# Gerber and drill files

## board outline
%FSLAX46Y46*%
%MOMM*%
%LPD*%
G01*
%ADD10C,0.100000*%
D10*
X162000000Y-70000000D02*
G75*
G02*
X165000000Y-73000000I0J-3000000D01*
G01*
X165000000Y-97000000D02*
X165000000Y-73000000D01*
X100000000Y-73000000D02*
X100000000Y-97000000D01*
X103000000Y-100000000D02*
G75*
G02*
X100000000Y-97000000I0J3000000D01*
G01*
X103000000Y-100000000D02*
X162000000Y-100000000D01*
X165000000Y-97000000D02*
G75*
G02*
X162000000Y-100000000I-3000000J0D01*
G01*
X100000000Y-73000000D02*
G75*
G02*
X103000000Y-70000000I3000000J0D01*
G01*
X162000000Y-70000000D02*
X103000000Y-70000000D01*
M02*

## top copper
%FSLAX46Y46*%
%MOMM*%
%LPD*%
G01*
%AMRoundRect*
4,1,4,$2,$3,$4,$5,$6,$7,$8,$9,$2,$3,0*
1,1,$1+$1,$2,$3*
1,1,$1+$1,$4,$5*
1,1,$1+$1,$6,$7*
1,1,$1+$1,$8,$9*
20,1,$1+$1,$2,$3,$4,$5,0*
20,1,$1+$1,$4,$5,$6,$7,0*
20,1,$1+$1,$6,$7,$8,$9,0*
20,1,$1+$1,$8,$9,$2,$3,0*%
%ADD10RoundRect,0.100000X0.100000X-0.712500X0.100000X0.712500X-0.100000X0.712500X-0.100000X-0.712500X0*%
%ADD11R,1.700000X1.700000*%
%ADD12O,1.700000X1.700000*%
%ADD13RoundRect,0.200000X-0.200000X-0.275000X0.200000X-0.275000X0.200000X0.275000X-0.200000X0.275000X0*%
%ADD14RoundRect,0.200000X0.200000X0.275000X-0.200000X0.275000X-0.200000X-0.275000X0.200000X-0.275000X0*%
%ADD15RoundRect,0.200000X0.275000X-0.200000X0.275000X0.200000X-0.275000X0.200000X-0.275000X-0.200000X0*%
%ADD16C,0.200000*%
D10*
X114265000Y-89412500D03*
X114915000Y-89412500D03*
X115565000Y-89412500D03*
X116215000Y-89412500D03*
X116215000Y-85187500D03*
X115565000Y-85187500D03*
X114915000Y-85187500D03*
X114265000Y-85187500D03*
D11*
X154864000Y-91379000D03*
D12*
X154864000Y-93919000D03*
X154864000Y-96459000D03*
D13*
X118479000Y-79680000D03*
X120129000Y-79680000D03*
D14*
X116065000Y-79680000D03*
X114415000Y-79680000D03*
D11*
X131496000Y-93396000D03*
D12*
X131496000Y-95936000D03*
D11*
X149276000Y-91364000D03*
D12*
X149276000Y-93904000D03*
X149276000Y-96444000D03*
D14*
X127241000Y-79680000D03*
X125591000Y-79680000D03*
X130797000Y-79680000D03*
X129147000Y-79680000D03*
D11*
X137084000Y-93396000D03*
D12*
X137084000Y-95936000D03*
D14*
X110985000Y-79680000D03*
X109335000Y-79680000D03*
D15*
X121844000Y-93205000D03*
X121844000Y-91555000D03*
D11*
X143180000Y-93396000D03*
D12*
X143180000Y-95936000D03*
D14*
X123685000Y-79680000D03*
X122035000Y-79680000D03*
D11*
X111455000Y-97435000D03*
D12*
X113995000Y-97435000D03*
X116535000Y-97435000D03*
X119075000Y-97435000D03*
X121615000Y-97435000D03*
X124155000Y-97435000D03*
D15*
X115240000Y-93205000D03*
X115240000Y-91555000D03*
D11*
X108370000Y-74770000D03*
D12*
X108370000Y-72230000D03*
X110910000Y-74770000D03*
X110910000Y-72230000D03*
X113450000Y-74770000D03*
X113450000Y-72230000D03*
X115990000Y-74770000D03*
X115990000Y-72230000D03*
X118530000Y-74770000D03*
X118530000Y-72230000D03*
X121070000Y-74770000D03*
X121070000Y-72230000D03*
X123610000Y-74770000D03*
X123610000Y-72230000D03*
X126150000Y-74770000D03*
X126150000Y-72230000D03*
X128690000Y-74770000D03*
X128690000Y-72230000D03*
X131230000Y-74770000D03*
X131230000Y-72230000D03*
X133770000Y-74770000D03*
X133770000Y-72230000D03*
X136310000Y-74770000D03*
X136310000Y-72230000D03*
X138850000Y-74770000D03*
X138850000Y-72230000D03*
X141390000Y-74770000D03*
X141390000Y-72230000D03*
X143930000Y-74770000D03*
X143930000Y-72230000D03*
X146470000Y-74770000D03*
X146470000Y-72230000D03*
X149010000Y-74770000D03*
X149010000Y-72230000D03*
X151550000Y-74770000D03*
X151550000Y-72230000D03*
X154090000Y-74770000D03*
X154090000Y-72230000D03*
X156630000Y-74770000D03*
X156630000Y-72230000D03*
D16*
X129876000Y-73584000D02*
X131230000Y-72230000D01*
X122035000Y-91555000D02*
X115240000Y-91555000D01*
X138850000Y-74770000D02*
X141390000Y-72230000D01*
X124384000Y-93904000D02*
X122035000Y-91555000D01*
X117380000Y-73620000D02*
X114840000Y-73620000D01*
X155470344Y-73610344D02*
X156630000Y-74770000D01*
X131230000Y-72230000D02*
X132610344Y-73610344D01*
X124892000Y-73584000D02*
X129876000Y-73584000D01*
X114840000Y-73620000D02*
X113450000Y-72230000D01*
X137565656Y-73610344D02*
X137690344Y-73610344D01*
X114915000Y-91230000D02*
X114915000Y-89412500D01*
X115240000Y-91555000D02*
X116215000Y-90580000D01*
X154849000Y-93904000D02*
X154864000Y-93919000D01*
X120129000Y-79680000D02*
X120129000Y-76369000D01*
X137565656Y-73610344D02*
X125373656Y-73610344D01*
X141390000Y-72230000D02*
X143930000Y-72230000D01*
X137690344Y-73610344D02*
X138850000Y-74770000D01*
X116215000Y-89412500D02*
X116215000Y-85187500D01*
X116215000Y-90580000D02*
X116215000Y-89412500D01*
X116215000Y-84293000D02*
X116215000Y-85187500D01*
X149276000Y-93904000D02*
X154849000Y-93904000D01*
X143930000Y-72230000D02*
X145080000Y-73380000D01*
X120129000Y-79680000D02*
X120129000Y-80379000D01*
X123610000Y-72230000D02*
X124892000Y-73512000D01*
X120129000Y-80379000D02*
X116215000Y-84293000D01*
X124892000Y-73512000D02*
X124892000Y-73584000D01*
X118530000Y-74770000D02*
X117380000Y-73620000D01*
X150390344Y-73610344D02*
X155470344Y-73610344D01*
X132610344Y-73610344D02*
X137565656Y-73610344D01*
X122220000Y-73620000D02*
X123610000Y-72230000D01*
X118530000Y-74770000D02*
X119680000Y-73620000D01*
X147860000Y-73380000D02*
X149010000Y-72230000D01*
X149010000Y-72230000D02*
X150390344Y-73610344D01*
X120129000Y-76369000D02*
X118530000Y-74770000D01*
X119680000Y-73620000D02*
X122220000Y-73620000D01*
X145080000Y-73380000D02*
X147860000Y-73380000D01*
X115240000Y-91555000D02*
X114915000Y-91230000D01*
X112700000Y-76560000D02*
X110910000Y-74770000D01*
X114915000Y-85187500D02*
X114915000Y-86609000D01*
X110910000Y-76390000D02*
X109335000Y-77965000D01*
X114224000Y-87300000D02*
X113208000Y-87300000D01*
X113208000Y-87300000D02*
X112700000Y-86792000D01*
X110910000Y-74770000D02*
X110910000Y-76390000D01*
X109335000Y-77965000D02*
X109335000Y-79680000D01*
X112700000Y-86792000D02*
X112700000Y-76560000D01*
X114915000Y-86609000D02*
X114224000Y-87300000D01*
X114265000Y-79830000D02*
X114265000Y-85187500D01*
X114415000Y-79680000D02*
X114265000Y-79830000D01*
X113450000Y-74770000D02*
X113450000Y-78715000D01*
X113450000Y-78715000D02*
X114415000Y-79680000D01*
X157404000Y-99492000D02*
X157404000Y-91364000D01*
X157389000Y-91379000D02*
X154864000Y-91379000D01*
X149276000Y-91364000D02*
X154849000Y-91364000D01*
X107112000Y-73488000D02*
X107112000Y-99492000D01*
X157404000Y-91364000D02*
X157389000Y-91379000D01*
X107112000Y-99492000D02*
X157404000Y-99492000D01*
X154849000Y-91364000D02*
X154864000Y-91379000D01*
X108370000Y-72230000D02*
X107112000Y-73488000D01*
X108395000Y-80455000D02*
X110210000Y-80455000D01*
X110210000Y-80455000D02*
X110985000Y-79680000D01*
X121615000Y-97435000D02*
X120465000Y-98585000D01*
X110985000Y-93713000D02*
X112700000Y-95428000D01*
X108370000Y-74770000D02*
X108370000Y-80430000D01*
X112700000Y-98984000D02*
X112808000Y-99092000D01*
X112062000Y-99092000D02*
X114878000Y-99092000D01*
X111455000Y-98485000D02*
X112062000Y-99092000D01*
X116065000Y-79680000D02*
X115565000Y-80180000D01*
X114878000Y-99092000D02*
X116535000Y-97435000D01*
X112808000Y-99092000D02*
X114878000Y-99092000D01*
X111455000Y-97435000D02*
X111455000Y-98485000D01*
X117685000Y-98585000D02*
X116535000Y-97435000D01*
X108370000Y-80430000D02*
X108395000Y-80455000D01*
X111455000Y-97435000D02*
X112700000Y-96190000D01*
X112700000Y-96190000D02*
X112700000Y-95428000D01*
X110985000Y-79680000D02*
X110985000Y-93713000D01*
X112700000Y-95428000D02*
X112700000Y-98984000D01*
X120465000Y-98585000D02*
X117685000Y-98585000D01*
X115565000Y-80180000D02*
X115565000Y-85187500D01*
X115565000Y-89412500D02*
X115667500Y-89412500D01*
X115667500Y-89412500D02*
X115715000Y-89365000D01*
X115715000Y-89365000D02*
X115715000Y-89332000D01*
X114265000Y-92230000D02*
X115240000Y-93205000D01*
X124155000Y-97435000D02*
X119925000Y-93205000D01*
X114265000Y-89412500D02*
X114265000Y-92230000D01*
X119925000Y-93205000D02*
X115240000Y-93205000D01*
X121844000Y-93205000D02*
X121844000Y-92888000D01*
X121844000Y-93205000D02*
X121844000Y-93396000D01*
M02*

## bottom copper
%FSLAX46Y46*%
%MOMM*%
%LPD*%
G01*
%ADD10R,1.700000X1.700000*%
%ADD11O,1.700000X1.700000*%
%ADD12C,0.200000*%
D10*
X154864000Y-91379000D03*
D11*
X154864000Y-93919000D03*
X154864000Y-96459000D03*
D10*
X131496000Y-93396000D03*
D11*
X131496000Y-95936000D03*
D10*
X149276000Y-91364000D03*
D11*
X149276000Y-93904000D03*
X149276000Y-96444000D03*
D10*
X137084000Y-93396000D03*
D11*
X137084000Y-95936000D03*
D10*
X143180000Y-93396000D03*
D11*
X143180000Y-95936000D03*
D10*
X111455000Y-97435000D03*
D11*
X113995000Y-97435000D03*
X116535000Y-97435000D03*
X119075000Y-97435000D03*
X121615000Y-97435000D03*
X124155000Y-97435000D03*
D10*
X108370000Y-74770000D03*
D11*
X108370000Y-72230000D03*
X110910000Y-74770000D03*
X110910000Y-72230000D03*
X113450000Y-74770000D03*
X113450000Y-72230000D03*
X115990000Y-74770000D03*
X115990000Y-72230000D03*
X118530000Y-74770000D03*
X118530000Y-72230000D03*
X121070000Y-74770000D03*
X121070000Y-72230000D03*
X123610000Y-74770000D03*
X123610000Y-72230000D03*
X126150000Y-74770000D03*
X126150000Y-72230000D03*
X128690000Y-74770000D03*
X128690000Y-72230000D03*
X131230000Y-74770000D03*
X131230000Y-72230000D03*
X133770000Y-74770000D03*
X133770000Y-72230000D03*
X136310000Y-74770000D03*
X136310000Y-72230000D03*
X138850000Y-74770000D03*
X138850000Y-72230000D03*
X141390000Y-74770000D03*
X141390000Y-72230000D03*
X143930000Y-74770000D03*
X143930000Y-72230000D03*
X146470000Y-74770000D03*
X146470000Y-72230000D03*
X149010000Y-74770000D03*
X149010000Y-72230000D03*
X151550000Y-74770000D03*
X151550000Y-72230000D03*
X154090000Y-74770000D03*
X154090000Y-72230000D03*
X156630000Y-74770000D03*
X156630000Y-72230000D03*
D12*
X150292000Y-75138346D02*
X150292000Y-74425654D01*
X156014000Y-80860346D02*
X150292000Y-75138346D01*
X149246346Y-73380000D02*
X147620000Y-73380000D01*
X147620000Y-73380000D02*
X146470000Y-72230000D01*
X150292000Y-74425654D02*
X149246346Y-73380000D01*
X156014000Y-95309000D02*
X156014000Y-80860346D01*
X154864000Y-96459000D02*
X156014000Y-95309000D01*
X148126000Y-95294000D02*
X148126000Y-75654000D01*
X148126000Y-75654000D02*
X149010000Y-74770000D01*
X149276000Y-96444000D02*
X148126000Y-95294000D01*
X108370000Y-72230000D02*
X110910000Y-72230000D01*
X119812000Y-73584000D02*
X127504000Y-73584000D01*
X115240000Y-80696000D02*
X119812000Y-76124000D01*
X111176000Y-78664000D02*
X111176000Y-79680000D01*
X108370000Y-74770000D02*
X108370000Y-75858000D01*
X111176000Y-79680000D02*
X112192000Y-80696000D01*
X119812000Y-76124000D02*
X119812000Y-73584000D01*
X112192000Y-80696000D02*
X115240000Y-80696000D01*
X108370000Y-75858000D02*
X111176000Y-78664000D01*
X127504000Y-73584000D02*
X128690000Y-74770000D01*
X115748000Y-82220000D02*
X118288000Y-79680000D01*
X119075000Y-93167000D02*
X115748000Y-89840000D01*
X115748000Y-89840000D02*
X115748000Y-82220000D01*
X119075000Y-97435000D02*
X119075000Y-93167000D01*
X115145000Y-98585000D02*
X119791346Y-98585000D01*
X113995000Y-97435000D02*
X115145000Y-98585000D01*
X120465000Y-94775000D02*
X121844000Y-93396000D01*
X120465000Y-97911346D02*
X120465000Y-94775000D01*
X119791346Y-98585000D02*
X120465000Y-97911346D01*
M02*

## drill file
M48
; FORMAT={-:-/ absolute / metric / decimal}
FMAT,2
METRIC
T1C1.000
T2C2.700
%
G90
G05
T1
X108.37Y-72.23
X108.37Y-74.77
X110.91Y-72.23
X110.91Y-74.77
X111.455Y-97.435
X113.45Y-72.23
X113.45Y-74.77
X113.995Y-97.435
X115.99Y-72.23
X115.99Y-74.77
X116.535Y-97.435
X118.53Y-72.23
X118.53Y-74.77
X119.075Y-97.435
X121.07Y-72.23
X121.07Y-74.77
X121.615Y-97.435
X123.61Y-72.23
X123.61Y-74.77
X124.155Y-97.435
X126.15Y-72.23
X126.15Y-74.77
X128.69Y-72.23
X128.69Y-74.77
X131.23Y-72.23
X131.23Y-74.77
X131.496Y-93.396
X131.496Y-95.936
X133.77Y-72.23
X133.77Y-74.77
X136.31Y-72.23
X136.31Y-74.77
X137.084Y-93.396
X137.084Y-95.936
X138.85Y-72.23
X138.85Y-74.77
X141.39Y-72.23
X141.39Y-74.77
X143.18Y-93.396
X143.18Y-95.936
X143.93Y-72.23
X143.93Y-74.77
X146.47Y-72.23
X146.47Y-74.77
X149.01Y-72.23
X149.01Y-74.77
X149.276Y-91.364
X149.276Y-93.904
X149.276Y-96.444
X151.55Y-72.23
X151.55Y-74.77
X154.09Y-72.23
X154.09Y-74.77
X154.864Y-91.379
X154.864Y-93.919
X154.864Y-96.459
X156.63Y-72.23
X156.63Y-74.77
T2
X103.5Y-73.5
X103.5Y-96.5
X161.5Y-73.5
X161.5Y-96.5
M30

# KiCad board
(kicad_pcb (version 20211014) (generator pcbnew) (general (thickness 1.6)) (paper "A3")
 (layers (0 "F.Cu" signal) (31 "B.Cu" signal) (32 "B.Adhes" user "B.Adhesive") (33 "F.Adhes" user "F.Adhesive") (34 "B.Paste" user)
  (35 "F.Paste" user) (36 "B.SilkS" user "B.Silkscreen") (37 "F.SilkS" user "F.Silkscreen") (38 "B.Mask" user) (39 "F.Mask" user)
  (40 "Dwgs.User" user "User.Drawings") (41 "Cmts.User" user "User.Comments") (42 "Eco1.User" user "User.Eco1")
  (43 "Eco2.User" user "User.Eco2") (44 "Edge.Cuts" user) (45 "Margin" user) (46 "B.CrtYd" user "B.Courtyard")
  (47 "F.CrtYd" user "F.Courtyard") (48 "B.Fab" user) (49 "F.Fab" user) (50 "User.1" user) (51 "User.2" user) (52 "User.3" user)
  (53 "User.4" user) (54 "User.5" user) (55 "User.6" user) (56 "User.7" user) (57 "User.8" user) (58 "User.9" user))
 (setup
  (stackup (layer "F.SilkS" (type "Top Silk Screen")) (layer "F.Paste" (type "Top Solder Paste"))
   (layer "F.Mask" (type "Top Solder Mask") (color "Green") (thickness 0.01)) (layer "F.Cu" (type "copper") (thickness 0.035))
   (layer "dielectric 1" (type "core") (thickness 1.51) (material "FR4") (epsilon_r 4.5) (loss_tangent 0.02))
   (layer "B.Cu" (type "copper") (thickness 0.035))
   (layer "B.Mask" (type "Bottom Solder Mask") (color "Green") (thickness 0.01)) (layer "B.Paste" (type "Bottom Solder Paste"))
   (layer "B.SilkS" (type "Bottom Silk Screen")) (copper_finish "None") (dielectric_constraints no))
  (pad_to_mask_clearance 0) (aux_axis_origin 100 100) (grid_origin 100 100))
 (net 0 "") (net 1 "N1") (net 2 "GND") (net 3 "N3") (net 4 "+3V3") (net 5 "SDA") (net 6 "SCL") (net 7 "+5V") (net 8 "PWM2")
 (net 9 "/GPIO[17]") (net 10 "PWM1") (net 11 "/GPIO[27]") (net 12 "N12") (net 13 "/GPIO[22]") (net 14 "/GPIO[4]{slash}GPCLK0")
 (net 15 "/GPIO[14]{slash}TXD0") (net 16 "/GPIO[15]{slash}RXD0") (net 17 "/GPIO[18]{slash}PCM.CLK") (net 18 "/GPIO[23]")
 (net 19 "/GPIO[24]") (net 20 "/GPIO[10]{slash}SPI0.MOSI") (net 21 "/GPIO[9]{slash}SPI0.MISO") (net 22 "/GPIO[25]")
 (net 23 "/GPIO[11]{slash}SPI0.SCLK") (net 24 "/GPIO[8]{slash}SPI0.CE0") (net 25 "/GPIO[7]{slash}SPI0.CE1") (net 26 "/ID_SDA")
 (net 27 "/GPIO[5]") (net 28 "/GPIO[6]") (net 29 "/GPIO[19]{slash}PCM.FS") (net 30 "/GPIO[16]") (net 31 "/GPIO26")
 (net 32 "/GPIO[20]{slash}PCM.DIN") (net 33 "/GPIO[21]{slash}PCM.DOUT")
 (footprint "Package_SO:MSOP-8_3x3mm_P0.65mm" (layer "F.Cu") (at 115.24 87.3 90)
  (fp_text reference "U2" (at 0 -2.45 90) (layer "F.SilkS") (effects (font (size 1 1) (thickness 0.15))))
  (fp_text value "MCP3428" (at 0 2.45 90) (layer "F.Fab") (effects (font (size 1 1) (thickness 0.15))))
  (pad "1" smd roundrect (at -2.1125 -0.975 90) (size 1.625 0.4) (layers "F.Cu" "F.Paste" "F.Mask") (roundrect_rratio 0.25) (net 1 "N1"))
  (pad "2" smd roundrect (at -2.1125 -0.325 90) (size 1.625 0.4) (layers "F.Cu" "F.Paste" "F.Mask") (roundrect_rratio 0.25) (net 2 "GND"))
  (pad "3" smd roundrect (at -2.1125 0.325 90) (size 1.625 0.4) (layers "F.Cu" "F.Paste" "F.Mask") (roundrect_rratio 0.25) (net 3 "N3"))
  (pad "4" smd roundrect (at -2.1125 0.975 90) (size 1.625 0.4) (layers "F.Cu" "F.Paste" "F.Mask") (roundrect_rratio 0.25) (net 2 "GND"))
  (pad "5" smd roundrect (at 2.1125 0.975 90) (size 1.625 0.4) (layers "F.Cu" "F.Paste" "F.Mask") (roundrect_rratio 0.25) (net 2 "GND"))
  (pad "6" smd roundrect (at 2.1125 0.325 90) (size 1.625 0.4) (layers "F.Cu" "F.Paste" "F.Mask") (roundrect_rratio 0.25) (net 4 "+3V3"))
  (pad "7" smd roundrect (at 2.1125 -0.325 90) (size 1.625 0.4) (layers "F.Cu" "F.Paste" "F.Mask") (roundrect_rratio 0.25) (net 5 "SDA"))
  (pad "8" smd roundrect (at 2.1125 -0.975 90) (size 1.625 0.4) (layers "F.Cu" "F.Paste" "F.Mask") (roundrect_rratio 0.25) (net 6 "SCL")))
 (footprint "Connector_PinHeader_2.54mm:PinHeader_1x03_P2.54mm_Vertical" (layer "F.Cu") (at 154.864 91.379)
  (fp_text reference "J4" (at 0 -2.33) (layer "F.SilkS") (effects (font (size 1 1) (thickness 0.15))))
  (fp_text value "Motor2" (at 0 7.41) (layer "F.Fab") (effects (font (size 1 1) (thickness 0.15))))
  (pad "1" thru_hole rect (at 0 0) (size 1.7 1.7) (drill 1) (layers *.Cu *.Mask) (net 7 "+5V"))
  (pad "2" thru_hole oval (at 0 2.54) (size 1.7 1.7) (drill 1) (layers *.Cu *.Mask) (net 2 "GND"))
  (pad "3" thru_hole oval (at 0 5.08) (size 1.7 1.7) (drill 1) (layers *.Cu *.Mask) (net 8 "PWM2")))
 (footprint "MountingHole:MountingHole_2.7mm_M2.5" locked (layer "F.Cu") (at 161.5 73.5)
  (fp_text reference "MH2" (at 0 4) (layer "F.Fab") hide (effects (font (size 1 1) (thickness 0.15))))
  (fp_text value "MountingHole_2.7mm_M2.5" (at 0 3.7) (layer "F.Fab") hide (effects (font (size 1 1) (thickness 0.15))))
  (pad "" np_thru_hole circle locked (at 0 0) (size 2.7 2.7) (drill 2.7) (layers *.Cu *.Mask)))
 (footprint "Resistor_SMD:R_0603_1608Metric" (layer "F.Cu") (at 119.304 79.68)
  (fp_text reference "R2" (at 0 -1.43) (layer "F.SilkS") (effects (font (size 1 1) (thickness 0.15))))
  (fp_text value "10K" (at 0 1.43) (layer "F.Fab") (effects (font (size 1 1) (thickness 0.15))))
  (pad "1" smd roundrect (at -0.825 0) (size 0.8 0.95) (layers "F.Cu" "F.Paste" "F.Mask") (roundrect_rratio 0.25) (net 3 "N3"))
  (pad "2" smd roundrect (at 0.825 0) (size 0.8 0.95) (layers "F.Cu" "F.Paste" "F.Mask") (roundrect_rratio 0.25) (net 2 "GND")))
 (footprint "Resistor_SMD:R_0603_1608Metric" (layer "F.Cu") (at 115.24 79.68 180)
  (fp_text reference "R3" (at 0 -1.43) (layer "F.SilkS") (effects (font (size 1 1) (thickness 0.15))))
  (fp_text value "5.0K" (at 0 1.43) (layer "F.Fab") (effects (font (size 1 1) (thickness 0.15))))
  (pad "1" smd roundrect (at -0.825 0 180) (size 0.8 0.95) (layers "F.Cu" "F.Paste" "F.Mask") (roundrect_rratio 0.25) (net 4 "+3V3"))
  (pad "2" smd roundrect (at 0.825 0 180) (size 0.8 0.95) (layers "F.Cu" "F.Paste" "F.Mask") (roundrect_rratio 0.25) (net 6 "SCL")))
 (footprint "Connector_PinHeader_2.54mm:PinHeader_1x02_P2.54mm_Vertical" (layer "F.Cu") (at 131.496 93.396)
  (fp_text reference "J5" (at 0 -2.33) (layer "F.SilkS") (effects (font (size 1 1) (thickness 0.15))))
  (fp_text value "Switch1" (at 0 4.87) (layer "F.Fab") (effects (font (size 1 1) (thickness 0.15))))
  (pad "1" thru_hole rect (at 0 0) (size 1.7 1.7) (drill 1) (layers *.Cu *.Mask) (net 4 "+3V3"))
  (pad "2" thru_hole oval (at 0 2.54) (size 1.7 1.7) (drill 1) (layers *.Cu *.Mask) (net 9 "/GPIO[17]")))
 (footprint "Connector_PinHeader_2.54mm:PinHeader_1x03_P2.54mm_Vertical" (layer "F.Cu") (at 149.276 91.364)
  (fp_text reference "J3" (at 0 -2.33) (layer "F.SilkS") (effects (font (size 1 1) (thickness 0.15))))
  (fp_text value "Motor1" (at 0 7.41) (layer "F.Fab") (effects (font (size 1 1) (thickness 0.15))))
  (pad "1" thru_hole rect (at 0 0) (size 1.7 1.7) (drill 1) (layers *.Cu *.Mask) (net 7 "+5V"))
  (pad "2" thru_hole oval (at 0 2.54) (size 1.7 1.7) (drill 1) (layers *.Cu *.Mask) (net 2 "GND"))
  (pad "3" thru_hole oval (at 0 5.08) (size 1.7 1.7) (drill 1) (layers *.Cu *.Mask) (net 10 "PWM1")))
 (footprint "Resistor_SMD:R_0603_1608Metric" (layer "F.Cu") (at 126.416 79.68 180)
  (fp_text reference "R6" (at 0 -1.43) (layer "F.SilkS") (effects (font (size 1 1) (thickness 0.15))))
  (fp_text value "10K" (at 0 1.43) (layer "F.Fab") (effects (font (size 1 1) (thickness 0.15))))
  (pad "1" smd roundrect (at -0.825 0 180) (size 0.8 0.95) (layers "F.Cu" "F.Paste" "F.Mask") (roundrect_rratio 0.25) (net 9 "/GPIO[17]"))
  (pad "2" smd roundrect (at 0.825 0 180) (size 0.8 0.95) (layers "F.Cu" "F.Paste" "F.Mask") (roundrect_rratio 0.25) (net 2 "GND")))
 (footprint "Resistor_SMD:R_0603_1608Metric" (layer "F.Cu") (at 129.972 79.68 180)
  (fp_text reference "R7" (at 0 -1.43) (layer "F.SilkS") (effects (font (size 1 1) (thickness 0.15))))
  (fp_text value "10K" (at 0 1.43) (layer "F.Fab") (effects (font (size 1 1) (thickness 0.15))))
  (pad "1" smd roundrect (at -0.825 0 180) (size 0.8 0.95) (layers "F.Cu" "F.Paste" "F.Mask") (roundrect_rratio 0.25) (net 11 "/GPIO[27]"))
  (pad "2" smd roundrect (at 0.825 0 180) (size 0.8 0.95) (layers "F.Cu" "F.Paste" "F.Mask") (roundrect_rratio 0.25) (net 2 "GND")))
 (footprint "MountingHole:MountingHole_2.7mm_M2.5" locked (layer "F.Cu") (at 103.5 96.5)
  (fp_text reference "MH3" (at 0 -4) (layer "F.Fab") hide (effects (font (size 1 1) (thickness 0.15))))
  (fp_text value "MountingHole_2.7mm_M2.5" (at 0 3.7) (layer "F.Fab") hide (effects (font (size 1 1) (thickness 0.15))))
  (pad "" np_thru_hole circle locked (at 0 0) (size 2.7 2.7) (drill 2.7) (layers *.Cu *.Mask)))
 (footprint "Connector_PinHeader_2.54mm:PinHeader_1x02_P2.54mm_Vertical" (layer "F.Cu") (at 137.084 93.396)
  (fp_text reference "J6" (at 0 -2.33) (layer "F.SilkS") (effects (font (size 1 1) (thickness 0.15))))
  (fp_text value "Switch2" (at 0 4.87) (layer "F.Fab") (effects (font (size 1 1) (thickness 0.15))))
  (pad "1" thru_hole rect (at 0 0) (size 1.7 1.7) (drill 1) (layers *.Cu *.Mask) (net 4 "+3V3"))
  (pad "2" thru_hole oval (at 0 2.54) (size 1.7 1.7) (drill 1) (layers *.Cu *.Mask) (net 11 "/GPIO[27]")))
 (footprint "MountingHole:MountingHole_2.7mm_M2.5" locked (layer "F.Cu") (at 103.5 73.5)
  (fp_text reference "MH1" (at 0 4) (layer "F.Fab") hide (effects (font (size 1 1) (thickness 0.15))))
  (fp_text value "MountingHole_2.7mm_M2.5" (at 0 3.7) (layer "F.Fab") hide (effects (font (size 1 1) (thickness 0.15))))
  (pad "" np_thru_hole circle locked (at 0 0) (size 2.7 2.7) (drill 2.7) (layers *.Cu *.Mask)))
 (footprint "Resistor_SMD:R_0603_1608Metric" (layer "F.Cu") (at 110.16 79.68 180)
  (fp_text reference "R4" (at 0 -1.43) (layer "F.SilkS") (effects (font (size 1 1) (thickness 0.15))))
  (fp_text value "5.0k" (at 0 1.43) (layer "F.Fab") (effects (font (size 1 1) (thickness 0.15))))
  (pad "1" smd roundrect (at -0.825 0 180) (size 0.8 0.95) (layers "F.Cu" "F.Paste" "F.Mask") (roundrect_rratio 0.25) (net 4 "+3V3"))
  (pad "2" smd roundrect (at 0.825 0 180) (size 0.8 0.95) (layers "F.Cu" "F.Paste" "F.Mask") (roundrect_rratio 0.25) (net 5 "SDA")))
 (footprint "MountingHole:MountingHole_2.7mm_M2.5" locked (layer "F.Cu") (at 161.5 96.5)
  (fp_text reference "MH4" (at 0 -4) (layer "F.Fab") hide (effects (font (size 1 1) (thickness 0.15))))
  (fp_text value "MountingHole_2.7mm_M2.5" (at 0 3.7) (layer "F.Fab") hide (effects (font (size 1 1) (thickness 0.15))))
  (pad "" np_thru_hole circle locked (at 0 0) (size 2.7 2.7) (drill 2.7) (layers *.Cu *.Mask)))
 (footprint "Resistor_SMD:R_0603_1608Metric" (layer "F.Cu") (at 121.844 92.38 90)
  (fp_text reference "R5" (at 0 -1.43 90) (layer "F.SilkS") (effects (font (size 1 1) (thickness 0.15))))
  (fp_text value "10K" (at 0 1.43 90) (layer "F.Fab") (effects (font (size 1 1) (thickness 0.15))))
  (pad "1" smd roundrect (at -0.825 0 90) (size 0.8 0.95) (layers "F.Cu" "F.Paste" "F.Mask") (roundrect_rratio 0.25) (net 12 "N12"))
  (pad "2" smd roundrect (at 0.825 0 90) (size 0.8 0.95) (layers "F.Cu" "F.Paste" "F.Mask") (roundrect_rratio 0.25) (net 2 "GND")))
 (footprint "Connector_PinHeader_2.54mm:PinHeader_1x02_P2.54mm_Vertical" (layer "F.Cu") (at 143.18 93.396)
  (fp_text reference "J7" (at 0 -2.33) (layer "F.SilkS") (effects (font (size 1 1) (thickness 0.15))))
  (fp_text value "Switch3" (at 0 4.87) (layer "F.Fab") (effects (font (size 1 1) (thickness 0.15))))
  (pad "1" thru_hole rect (at 0 0) (size 1.7 1.7) (drill 1) (layers *.Cu *.Mask) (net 4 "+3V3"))
  (pad "2" thru_hole oval (at 0 2.54) (size 1.7 1.7) (drill 1) (layers *.Cu *.Mask) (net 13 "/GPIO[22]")))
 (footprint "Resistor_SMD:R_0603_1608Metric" (layer "F.Cu") (at 122.86 79.68 180)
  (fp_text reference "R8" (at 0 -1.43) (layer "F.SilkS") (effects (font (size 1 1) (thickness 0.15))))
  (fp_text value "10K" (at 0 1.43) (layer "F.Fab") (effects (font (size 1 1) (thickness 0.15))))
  (pad "1" smd roundrect (at -0.825 0 180) (size 0.8 0.95) (layers "F.Cu" "F.Paste" "F.Mask") (roundrect_rratio 0.25) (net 13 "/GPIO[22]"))
  (pad "2" smd roundrect (at 0.825 0 180) (size 0.8 0.95) (layers "F.Cu" "F.Paste" "F.Mask") (roundrect_rratio 0.25) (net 2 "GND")))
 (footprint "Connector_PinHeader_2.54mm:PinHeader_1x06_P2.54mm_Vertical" (layer "F.Cu") (at 111.455 97.435 90)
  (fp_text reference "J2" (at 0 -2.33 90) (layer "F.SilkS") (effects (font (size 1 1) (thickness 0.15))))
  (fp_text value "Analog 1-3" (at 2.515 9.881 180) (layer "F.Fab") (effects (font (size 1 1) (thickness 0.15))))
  (pad "1" thru_hole rect (at 0 0 90) (size 1.7 1.7) (drill 1) (layers *.Cu *.Mask) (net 4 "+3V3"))
  (pad "2" thru_hole oval (at 0 2.54 90) (size 1.7 1.7) (drill 1) (layers *.Cu *.Mask) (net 12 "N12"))
  (pad "3" thru_hole oval (at 0 5.08 90) (size 1.7 1.7) (drill 1) (layers *.Cu *.Mask) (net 4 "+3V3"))
  (pad "4" thru_hole oval (at 0 7.62 90) (size 1.7 1.7) (drill 1) (layers *.Cu *.Mask) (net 3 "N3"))
  (pad "5" thru_hole oval (at 0 10.16 90) (size 1.7 1.7) (drill 1) (layers *.Cu *.Mask) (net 4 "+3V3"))
  (pad "6" thru_hole oval (at 0 12.7 90) (size 1.7 1.7) (drill 1) (layers *.Cu *.Mask) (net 1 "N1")))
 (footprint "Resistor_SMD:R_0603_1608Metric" (layer "F.Cu") (at 115.24 92.38 90)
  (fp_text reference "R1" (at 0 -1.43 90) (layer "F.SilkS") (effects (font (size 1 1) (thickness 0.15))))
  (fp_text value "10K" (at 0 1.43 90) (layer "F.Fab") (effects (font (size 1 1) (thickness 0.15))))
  (pad "1" smd roundrect (at -0.825 0 90) (size 0.8 0.95) (layers "F.Cu" "F.Paste" "F.Mask") (roundrect_rratio 0.25) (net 1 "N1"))
  (pad "2" smd roundrect (at 0.825 0 90) (size 0.8 0.95) (layers "F.Cu" "F.Paste" "F.Mask") (roundrect_rratio 0.25) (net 2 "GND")))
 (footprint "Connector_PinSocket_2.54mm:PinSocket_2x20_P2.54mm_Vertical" (layer "B.Cu") (at 108.37 74.77 -90)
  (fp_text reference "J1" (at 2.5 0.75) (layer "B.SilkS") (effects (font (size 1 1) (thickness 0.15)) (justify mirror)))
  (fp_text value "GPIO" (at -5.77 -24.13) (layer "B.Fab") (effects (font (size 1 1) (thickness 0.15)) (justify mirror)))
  (pad "1" thru_hole rect locked (at 0 0 270) (size 1.7 1.7) (drill 1) (layers *.Cu *.Mask) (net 4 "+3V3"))
  (pad "2" thru_hole oval locked (at -2.54 0 270) (size 1.7 1.7) (drill 1) (layers *.Cu *.Mask) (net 7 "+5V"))
  (pad "3" thru_hole oval locked (at 0 -2.54 270) (size 1.7 1.7) (drill 1) (layers *.Cu *.Mask) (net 5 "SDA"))
  (pad "4" thru_hole oval locked (at -2.54 -2.54 270) (size 1.7 1.7) (drill 1) (layers *.Cu *.Mask) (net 7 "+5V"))
  (pad "5" thru_hole oval locked (at 0 -5.08 270) (size 1.7 1.7) (drill 1) (layers *.Cu *.Mask) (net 6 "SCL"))
  (pad "6" thru_hole oval locked (at -2.54 -5.08 270) (size 1.7 1.7) (drill 1) (layers *.Cu *.Mask) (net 2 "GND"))
  (pad "7" thru_hole oval locked (at 0 -7.62 270) (size 1.7 1.7) (drill 1) (layers *.Cu *.Mask) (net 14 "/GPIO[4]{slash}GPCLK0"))
  (pad "8" thru_hole oval locked (at -2.54 -7.62 270) (size 1.7 1.7) (drill 1) (layers *.Cu *.Mask) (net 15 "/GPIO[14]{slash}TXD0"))
  (pad "9" thru_hole oval locked (at 0 -10.16 270) (size 1.7 1.7) (drill 1) (layers *.Cu *.Mask) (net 2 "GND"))
  (pad "10" thru_hole oval locked (at -2.54 -10.16 270) (size 1.7 1.7) (drill 1) (layers *.Cu *.Mask) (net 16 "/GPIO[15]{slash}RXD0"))
  (pad "11" thru_hole oval locked (at 0 -12.7 270) (size 1.7 1.7) (drill 1) (layers *.Cu *.Mask) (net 9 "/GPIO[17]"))
  (pad "12" thru_hole oval locked (at -2.54 -12.7 270) (size 1.7 1.7) (drill 1) (layers *.Cu *.Mask) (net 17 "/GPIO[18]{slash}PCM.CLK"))
  (pad "13" thru_hole oval locked (at 0 -15.24 270) (size 1.7 1.7) (drill 1) (layers *.Cu *.Mask) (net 11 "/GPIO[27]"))
  (pad "14" thru_hole oval locked (at -2.54 -15.24 270) (size 1.7 1.7) (drill 1) (layers *.Cu *.Mask) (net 2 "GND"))
  (pad "15" thru_hole oval locked (at 0 -17.78 270) (size 1.7 1.7) (drill 1) (layers *.Cu *.Mask) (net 13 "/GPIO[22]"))
  (pad "16" thru_hole oval locked (at -2.54 -17.78 270) (size 1.7 1.7) (drill 1) (layers *.Cu *.Mask) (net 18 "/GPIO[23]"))
  (pad "17" thru_hole oval locked (at 0 -20.32 270) (size 1.7 1.7) (drill 1) (layers *.Cu *.Mask) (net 4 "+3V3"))
  (pad "18" thru_hole oval locked (at -2.54 -20.32 270) (size 1.7 1.7) (drill 1) (layers *.Cu *.Mask) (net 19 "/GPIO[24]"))
  (pad "19" thru_hole oval locked (at 0 -22.86 270) (size 1.7 1.7) (drill 1) (layers *.Cu *.Mask) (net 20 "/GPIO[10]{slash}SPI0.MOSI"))
  (pad "20" thru_hole oval locked (at -2.54 -22.86 270) (size 1.7 1.7) (drill 1) (layers *.Cu *.Mask) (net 2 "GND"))
  (pad "21" thru_hole oval locked (at 0 -25.4 270) (size 1.7 1.7) (drill 1) (layers *.Cu *.Mask) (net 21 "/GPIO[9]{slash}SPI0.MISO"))
  (pad "22" thru_hole oval locked (at -2.54 -25.4 270) (size 1.7 1.7) (drill 1) (layers *.Cu *.Mask) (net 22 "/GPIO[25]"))
  (pad "23" thru_hole oval locked (at 0 -27.94 270) (size 1.7 1.7) (drill 1) (layers *.Cu *.Mask) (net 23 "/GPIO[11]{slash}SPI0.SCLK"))
  (pad "24" thru_hole oval locked (at -2.54 -27.94 270) (size 1.7 1.7) (drill 1) (layers *.Cu *.Mask) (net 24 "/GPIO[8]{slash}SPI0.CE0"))
  (pad "25" thru_hole oval locked (at 0 -30.48 270) (size 1.7 1.7) (drill 1) (layers *.Cu *.Mask) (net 2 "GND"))
  (pad "26" thru_hole oval locked (at -2.54 -30.48 270) (size 1.7 1.7) (drill 1) (layers *.Cu *.Mask) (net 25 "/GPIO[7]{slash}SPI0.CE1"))
  (pad "27" thru_hole oval locked (at 0 -33.02 270) (size 1.7 1.7) (drill 1) (layers *.Cu *.Mask) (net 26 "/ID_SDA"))
  (pad "28" thru_hole oval locked (at -2.54 -33.02 270) (size 1.7 1.7) (drill 1) (layers *.Cu *.Mask) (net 2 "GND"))
  (pad "29" thru_hole oval locked (at 0 -35.56 270) (size 1.7 1.7) (drill 1) (layers *.Cu *.Mask) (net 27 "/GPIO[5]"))
  (pad "30" thru_hole oval locked (at -2.54 -35.56 270) (size 1.7 1.7) (drill 1) (layers *.Cu *.Mask) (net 2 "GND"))
  (pad "31" thru_hole oval locked (at 0 -38.1 270) (size 1.7 1.7) (drill 1) (layers *.Cu *.Mask) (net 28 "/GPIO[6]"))
  (pad "32" thru_hole oval locked (at -2.54 -38.1 270) (size 1.7 1.7) (drill 1) (layers *.Cu *.Mask) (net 8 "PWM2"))
  (pad "33" thru_hole oval locked (at 0 -40.64 270) (size 1.7 1.7) (drill 1) (layers *.Cu *.Mask) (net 10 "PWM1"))
  (pad "34" thru_hole oval locked (at -2.54 -40.64 270) (size 1.7 1.7) (drill 1) (layers *.Cu *.Mask) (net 2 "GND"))
  (pad "35" thru_hole oval locked (at 0 -43.18 270) (size 1.7 1.7) (drill 1) (layers *.Cu *.Mask) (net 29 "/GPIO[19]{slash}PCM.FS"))
  (pad "36" thru_hole oval locked (at -2.54 -43.18 270) (size 1.7 1.7) (drill 1) (layers *.Cu *.Mask) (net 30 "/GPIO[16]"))
  (pad "37" thru_hole oval locked (at 0 -45.72 270) (size 1.7 1.7) (drill 1) (layers *.Cu *.Mask) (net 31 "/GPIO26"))
  (pad "38" thru_hole oval locked (at -2.54 -45.72 270) (size 1.7 1.7) (drill 1) (layers *.Cu *.Mask) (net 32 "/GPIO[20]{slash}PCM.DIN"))
  (pad "39" thru_hole oval locked (at 0 -48.26 270) (size 1.7 1.7) (drill 1) (layers *.Cu *.Mask) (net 2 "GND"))
  (pad "40" thru_hole oval locked (at -2.54 -48.26 270) (size 1.7 1.7) (drill 1) (layers *.Cu *.Mask) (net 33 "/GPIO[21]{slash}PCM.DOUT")))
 (gr_arc (start 162 70) (mid 164.12132 70.87868) (end 165 73) (layer "Edge.Cuts") (width 0.1))
 (gr_line (start 165 97) (end 165 73) (layer "Edge.Cuts") (width 0.1))
 (gr_line (start 100 73) (end 100 97) (layer "Edge.Cuts") (width 0.1))
 (gr_arc (start 103 100) (mid 100.87868 99.12132) (end 100 97) (layer "Edge.Cuts") (width 0.1))
 (gr_line (start 103 100) (end 162 100) (layer "Edge.Cuts") (width 0.1))
 (gr_arc (start 165 97) (mid 164.12132 99.12132) (end 162 100) (layer "Edge.Cuts") (width 0.1))
 (gr_arc (start 100 73) (mid 100.87868 70.87868) (end 103 70) (layer "Edge.Cuts") (width 0.1))
 (gr_line (start 162 70) (end 103 70) (layer "Edge.Cuts") (width 0.1))
 (segment (start 129.876 73.584) (end 131.23 72.23) (width 0.2) (layer "F.Cu") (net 2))
 (segment (start 122.035 91.555) (end 115.24 91.555) (width 0.2) (layer "F.Cu") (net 2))
 (segment (start 138.85 74.77) (end 141.39 72.23) (width 0.2) (layer "F.Cu") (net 2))
 (segment (start 124.384 93.904) (end 122.035 91.555) (width 0.2) (layer "F.Cu") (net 2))
 (segment (start 117.38 73.62) (end 114.84 73.62) (width 0.2) (layer "F.Cu") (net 2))
 (segment (start 155.470344 73.610344) (end 156.63 74.77) (width 0.2) (layer "F.Cu") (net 2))
 (segment (start 131.23 72.23) (end 132.610344 73.610344) (width 0.2) (layer "F.Cu") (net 2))
 (segment (start 124.892 73.584) (end 129.876 73.584) (width 0.2) (layer "F.Cu") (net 2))
 (segment (start 114.84 73.62) (end 113.45 72.23) (width 0.2) (layer "F.Cu") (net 2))
 (segment (start 137.565656 73.610344) (end 137.690344 73.610344) (width 0.2) (layer "F.Cu") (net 2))
 (segment (start 114.915 91.23) (end 114.915 89.4125) (width 0.2) (layer "F.Cu") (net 2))
 (segment (start 115.24 91.555) (end 116.215 90.58) (width 0.2) (layer "F.Cu") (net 2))
 (segment (start 154.849 93.904) (end 154.864 93.919) (width 0.2) (layer "F.Cu") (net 2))
 (segment (start 120.129 79.68) (end 120.129 76.369) (width 0.2) (layer "F.Cu") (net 2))
 (segment (start 137.565656 73.610344) (end 125.373656 73.610344) (width 0.2) (layer "F.Cu") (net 2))
 (segment (start 141.39 72.23) (end 143.93 72.23) (width 0.2) (layer "F.Cu") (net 2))
 (segment (start 137.690344 73.610344) (end 138.85 74.77) (width 0.2) (layer "F.Cu") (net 2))
 (segment (start 116.215 89.4125) (end 116.215 85.1875) (width 0.2) (layer "F.Cu") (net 2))
 (segment (start 116.215 90.58) (end 116.215 89.4125) (width 0.2) (layer "F.Cu") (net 2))
 (segment (start 116.215 84.293) (end 116.215 85.1875) (width 0.2) (layer "F.Cu") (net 2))
 (segment (start 149.276 93.904) (end 154.849 93.904) (width 0.2) (layer "F.Cu") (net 2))
 (segment (start 143.93 72.23) (end 145.08 73.38) (width 0.2) (layer "F.Cu") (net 2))
 (segment (start 120.129 79.68) (end 120.129 80.379) (width 0.2) (layer "F.Cu") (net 2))
 (segment (start 123.61 72.23) (end 124.892 73.512) (width 0.2) (layer "F.Cu") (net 2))
 (segment (start 120.129 80.379) (end 116.215 84.293) (width 0.2) (layer "F.Cu") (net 2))
 (segment (start 124.892 73.512) (end 124.892 73.584) (width 0.2) (layer "F.Cu") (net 2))
 (segment (start 118.53 74.77) (end 117.38 73.62) (width 0.2) (layer "F.Cu") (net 2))
 (segment (start 150.390344 73.610344) (end 155.470344 73.610344) (width 0.2) (layer "F.Cu") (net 2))
 (segment (start 132.610344 73.610344) (end 137.565656 73.610344) (width 0.2) (layer "F.Cu") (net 2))
 (segment (start 122.22 73.62) (end 123.61 72.23) (width 0.2) (layer "F.Cu") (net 2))
 (segment (start 118.53 74.77) (end 119.68 73.62) (width 0.2) (layer "F.Cu") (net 2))
 (segment (start 147.86 73.38) (end 149.01 72.23) (width 0.2) (layer "F.Cu") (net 2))
 (segment (start 149.01 72.23) (end 150.390344 73.610344) (width 0.2) (layer "F.Cu") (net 2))
 (segment (start 120.129 76.369) (end 118.53 74.77) (width 0.2) (layer "F.Cu") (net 2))
 (segment (start 119.68 73.62) (end 122.22 73.62) (width 0.2) (layer "F.Cu") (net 2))
 (segment (start 145.08 73.38) (end 147.86 73.38) (width 0.2) (layer "F.Cu") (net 2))
 (segment (start 115.24 91.555) (end 114.915 91.23) (width 0.2) (layer "F.Cu") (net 2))
 (segment (start 112.7 76.56) (end 110.91 74.77) (width 0.2) (layer "F.Cu") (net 5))
 (segment (start 114.915 85.1875) (end 114.915 86.609) (width 0.2) (layer "F.Cu") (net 5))
 (segment (start 110.91 76.39) (end 109.335 77.965) (width 0.2) (layer "F.Cu") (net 5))
 (segment (start 114.224 87.3) (end 113.208 87.3) (width 0.2) (layer "F.Cu") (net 5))
 (segment (start 113.208 87.3) (end 112.7 86.792) (width 0.2) (layer "F.Cu") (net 5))
 (segment (start 110.91 74.77) (end 110.91 76.39) (width 0.2) (layer "F.Cu") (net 5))
 (segment (start 109.335 77.965) (end 109.335 79.68) (width 0.2) (layer "F.Cu") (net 5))
 (segment (start 112.7 86.792) (end 112.7 76.56) (width 0.2) (layer "F.Cu") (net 5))
 (segment (start 114.915 86.609) (end 114.224 87.3) (width 0.2) (layer "F.Cu") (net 5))
 (segment (start 114.265 79.83) (end 114.265 85.1875) (width 0.2) (layer "F.Cu") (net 6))
 (segment (start 114.415 79.68) (end 114.265 79.83) (width 0.2) (layer "F.Cu") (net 6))
 (segment (start 113.45 74.77) (end 113.45 78.715) (width 0.2) (layer "F.Cu") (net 6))
 (segment (start 113.45 78.715) (end 114.415 79.68) (width 0.2) (layer "F.Cu") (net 6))
 (segment (start 150.292 75.138346) (end 150.292 74.425654) (width 0.2) (layer "B.Cu") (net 8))
 (segment (start 156.014 80.860346) (end 150.292 75.138346) (width 0.2) (layer "B.Cu") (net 8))
 (segment (start 149.246346 73.38) (end 147.62 73.38) (width 0.2) (layer "B.Cu") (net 8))
 (segment (start 147.62 73.38) (end 146.47 72.23) (width 0.2) (layer "B.Cu") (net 8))
 (segment (start 150.292 74.425654) (end 149.246346 73.38) (width 0.2) (layer "B.Cu") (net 8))
 (segment (start 156.014 95.309) (end 156.014 80.860346) (width 0.2) (layer "B.Cu") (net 8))
 (segment (start 154.864 96.459) (end 156.014 95.309) (width 0.2) (layer "B.Cu") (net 8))
 (segment (start 148.126 95.294) (end 148.126 75.654) (width 0.2) (layer "B.Cu") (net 10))
 (segment (start 148.126 75.654) (end 149.01 74.77) (width 0.2) (layer "B.Cu") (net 10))
 (segment (start 149.276 96.444) (end 148.126 95.294) (width 0.2) (layer "B.Cu") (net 10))
 (segment (start 157.404 99.492) (end 157.404 91.364) (width 0.2) (layer "F.Cu") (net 7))
 (segment (start 157.389 91.379) (end 154.864 91.379) (width 0.2) (layer "F.Cu") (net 7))
 (segment (start 149.276 91.364) (end 154.849 91.364) (width 0.2) (layer "F.Cu") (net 7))
 (segment (start 107.112 73.488) (end 107.112 99.492) (width 0.2) (layer "F.Cu") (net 7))
 (segment (start 157.404 91.364) (end 157.389 91.379) (width 0.2) (layer "F.Cu") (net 7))
 (segment (start 107.112 99.492) (end 157.404 99.492) (width 0.2) (layer "F.Cu") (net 7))
 (segment (start 154.849 91.364) (end 154.864 91.379) (width 0.2) (layer "F.Cu") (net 7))
 (segment (start 108.37 72.23) (end 107.112 73.488) (width 0.2) (layer "F.Cu") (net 7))
 (segment (start 108.37 72.23) (end 110.91 72.23) (width 0.2) (layer "B.Cu") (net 7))
 (segment (start 108.395 80.455) (end 110.21 80.455) (width 0.2) (layer "F.Cu") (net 4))
 (segment (start 110.21 80.455) (end 110.985 79.68) (width 0.2) (layer "F.Cu") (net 4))
 (segment (start 121.615 97.435) (end 120.465 98.585) (width 0.2) (layer "F.Cu") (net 4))
 (segment (start 110.985 93.713) (end 112.7 95.428) (width 0.2) (layer "F.Cu") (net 4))
 (segment (start 108.37 74.77) (end 108.37 80.43) (width 0.2) (layer "F.Cu") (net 4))
 (segment (start 112.7 98.984) (end 112.808 99.092) (width 0.2) (layer "F.Cu") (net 4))
 (segment (start 112.062 99.092) (end 114.878 99.092) (width 0.2) (layer "F.Cu") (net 4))
 (segment (start 111.455 98.485) (end 112.062 99.092) (width 0.2) (layer "F.Cu") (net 4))
 (segment (start 116.065 79.68) (end 115.565 80.18) (width 0.2) (layer "F.Cu") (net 4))
 (segment (start 114.878 99.092) (end 116.535 97.435) (width 0.2) (layer "F.Cu") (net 4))
 (segment (start 112.808 99.092) (end 114.878 99.092) (width 0.2) (layer "F.Cu") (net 4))
 (segment (start 111.455 97.435) (end 111.455 98.485) (width 0.2) (layer "F.Cu") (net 4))
 (segment (start 117.685 98.585) (end 116.535 97.435) (width 0.2) (layer "F.Cu") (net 4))
 (segment (start 108.37 80.43) (end 108.395 80.455) (width 0.2) (layer "F.Cu") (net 4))
 (segment (start 111.455 97.435) (end 112.7 96.19) (width 0.2) (layer "F.Cu") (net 4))
 (segment (start 112.7 96.19) (end 112.7 95.428) (width 0.2) (layer "F.Cu") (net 4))
 (segment (start 110.985 79.68) (end 110.985 93.713) (width 0.2) (layer "F.Cu") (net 4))
 (segment (start 112.7 95.428) (end 112.7 98.984) (width 0.2) (layer "F.Cu") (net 4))
 (segment (start 120.465 98.585) (end 117.685 98.585) (width 0.2) (layer "F.Cu") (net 4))
 (segment (start 115.565 80.18) (end 115.565 85.1875) (width 0.2) (layer "F.Cu") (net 4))
 (segment (start 119.812 73.584) (end 127.504 73.584) (width 0.2) (layer "B.Cu") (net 4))
 (segment (start 115.24 80.696) (end 119.812 76.124) (width 0.2) (layer "B.Cu") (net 4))
 (segment (start 111.176 78.664) (end 111.176 79.68) (width 0.2) (layer "B.Cu") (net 4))
 (segment (start 108.37 74.77) (end 108.37 75.858) (width 0.2) (layer "B.Cu") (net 4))
 (segment (start 111.176 79.68) (end 112.192 80.696) (width 0.2) (layer "B.Cu") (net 4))
 (segment (start 119.812 76.124) (end 119.812 73.584) (width 0.2) (layer "B.Cu") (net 4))
 (segment (start 112.192 80.696) (end 115.24 80.696) (width 0.2) (layer "B.Cu") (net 4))
 (segment (start 108.37 75.858) (end 111.176 78.664) (width 0.2) (layer "B.Cu") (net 4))
 (segment (start 127.504 73.584) (end 128.69 74.77) (width 0.2) (layer "B.Cu") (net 4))
 (segment (start 115.565 89.4125) (end 115.6675 89.4125) (width 0.2) (layer "F.Cu") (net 3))
 (segment (start 115.6675 89.4125) (end 115.715 89.365) (width 0.2) (layer "F.Cu") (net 3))
 (segment (start 115.715 89.365) (end 115.715 89.332) (width 0.2) (layer "F.Cu") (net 3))
 (segment (start 115.748 82.22) (end 118.288 79.68) (width 0.2) (layer "B.Cu") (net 3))
 (segment (start 119.075 93.167) (end 115.748 89.84) (width 0.2) (layer "B.Cu") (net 3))
 (segment (start 115.748 89.84) (end 115.748 82.22) (width 0.2) (layer "B.Cu") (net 3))
 (segment (start 119.075 97.435) (end 119.075 93.167) (width 0.2) (layer "B.Cu") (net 3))
 (segment (start 114.265 92.23) (end 115.24 93.205) (width 0.2) (layer "F.Cu") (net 1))
 (segment (start 124.155 97.435) (end 119.925 93.205) (width 0.2) (layer "F.Cu") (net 1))
 (segment (start 114.265 89.4125) (end 114.265 92.23) (width 0.2) (layer "F.Cu") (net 1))
 (segment (start 119.925 93.205) (end 115.24 93.205) (width 0.2) (layer "F.Cu") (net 1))
 (segment (start 121.844 93.205) (end 121.844 92.888) (width 0.2) (layer "F.Cu") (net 12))
 (segment (start 121.844 93.205) (end 121.844 93.396) (width 0.2) (layer "F.Cu") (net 12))
 (segment (start 115.145 98.585) (end 119.791346 98.585) (width 0.2) (layer "B.Cu") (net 12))
 (segment (start 113.995 97.435) (end 115.145 98.585) (width 0.2) (layer "B.Cu") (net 12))
 (segment (start 120.465 94.775) (end 121.844 93.396) (width 0.2) (layer "B.Cu") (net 12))
 (segment (start 120.465 97.911346) (end 120.465 94.775) (width 0.2) (layer "B.Cu") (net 12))
 (segment (start 119.791346 98.585) (end 120.465 97.911346) (width 0.2) (layer "B.Cu") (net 12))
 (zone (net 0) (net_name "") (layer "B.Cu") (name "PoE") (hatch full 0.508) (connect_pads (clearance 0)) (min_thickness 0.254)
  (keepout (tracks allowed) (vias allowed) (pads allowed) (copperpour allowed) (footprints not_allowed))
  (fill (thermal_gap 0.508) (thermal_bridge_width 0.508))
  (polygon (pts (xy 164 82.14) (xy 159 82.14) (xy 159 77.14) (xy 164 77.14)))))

